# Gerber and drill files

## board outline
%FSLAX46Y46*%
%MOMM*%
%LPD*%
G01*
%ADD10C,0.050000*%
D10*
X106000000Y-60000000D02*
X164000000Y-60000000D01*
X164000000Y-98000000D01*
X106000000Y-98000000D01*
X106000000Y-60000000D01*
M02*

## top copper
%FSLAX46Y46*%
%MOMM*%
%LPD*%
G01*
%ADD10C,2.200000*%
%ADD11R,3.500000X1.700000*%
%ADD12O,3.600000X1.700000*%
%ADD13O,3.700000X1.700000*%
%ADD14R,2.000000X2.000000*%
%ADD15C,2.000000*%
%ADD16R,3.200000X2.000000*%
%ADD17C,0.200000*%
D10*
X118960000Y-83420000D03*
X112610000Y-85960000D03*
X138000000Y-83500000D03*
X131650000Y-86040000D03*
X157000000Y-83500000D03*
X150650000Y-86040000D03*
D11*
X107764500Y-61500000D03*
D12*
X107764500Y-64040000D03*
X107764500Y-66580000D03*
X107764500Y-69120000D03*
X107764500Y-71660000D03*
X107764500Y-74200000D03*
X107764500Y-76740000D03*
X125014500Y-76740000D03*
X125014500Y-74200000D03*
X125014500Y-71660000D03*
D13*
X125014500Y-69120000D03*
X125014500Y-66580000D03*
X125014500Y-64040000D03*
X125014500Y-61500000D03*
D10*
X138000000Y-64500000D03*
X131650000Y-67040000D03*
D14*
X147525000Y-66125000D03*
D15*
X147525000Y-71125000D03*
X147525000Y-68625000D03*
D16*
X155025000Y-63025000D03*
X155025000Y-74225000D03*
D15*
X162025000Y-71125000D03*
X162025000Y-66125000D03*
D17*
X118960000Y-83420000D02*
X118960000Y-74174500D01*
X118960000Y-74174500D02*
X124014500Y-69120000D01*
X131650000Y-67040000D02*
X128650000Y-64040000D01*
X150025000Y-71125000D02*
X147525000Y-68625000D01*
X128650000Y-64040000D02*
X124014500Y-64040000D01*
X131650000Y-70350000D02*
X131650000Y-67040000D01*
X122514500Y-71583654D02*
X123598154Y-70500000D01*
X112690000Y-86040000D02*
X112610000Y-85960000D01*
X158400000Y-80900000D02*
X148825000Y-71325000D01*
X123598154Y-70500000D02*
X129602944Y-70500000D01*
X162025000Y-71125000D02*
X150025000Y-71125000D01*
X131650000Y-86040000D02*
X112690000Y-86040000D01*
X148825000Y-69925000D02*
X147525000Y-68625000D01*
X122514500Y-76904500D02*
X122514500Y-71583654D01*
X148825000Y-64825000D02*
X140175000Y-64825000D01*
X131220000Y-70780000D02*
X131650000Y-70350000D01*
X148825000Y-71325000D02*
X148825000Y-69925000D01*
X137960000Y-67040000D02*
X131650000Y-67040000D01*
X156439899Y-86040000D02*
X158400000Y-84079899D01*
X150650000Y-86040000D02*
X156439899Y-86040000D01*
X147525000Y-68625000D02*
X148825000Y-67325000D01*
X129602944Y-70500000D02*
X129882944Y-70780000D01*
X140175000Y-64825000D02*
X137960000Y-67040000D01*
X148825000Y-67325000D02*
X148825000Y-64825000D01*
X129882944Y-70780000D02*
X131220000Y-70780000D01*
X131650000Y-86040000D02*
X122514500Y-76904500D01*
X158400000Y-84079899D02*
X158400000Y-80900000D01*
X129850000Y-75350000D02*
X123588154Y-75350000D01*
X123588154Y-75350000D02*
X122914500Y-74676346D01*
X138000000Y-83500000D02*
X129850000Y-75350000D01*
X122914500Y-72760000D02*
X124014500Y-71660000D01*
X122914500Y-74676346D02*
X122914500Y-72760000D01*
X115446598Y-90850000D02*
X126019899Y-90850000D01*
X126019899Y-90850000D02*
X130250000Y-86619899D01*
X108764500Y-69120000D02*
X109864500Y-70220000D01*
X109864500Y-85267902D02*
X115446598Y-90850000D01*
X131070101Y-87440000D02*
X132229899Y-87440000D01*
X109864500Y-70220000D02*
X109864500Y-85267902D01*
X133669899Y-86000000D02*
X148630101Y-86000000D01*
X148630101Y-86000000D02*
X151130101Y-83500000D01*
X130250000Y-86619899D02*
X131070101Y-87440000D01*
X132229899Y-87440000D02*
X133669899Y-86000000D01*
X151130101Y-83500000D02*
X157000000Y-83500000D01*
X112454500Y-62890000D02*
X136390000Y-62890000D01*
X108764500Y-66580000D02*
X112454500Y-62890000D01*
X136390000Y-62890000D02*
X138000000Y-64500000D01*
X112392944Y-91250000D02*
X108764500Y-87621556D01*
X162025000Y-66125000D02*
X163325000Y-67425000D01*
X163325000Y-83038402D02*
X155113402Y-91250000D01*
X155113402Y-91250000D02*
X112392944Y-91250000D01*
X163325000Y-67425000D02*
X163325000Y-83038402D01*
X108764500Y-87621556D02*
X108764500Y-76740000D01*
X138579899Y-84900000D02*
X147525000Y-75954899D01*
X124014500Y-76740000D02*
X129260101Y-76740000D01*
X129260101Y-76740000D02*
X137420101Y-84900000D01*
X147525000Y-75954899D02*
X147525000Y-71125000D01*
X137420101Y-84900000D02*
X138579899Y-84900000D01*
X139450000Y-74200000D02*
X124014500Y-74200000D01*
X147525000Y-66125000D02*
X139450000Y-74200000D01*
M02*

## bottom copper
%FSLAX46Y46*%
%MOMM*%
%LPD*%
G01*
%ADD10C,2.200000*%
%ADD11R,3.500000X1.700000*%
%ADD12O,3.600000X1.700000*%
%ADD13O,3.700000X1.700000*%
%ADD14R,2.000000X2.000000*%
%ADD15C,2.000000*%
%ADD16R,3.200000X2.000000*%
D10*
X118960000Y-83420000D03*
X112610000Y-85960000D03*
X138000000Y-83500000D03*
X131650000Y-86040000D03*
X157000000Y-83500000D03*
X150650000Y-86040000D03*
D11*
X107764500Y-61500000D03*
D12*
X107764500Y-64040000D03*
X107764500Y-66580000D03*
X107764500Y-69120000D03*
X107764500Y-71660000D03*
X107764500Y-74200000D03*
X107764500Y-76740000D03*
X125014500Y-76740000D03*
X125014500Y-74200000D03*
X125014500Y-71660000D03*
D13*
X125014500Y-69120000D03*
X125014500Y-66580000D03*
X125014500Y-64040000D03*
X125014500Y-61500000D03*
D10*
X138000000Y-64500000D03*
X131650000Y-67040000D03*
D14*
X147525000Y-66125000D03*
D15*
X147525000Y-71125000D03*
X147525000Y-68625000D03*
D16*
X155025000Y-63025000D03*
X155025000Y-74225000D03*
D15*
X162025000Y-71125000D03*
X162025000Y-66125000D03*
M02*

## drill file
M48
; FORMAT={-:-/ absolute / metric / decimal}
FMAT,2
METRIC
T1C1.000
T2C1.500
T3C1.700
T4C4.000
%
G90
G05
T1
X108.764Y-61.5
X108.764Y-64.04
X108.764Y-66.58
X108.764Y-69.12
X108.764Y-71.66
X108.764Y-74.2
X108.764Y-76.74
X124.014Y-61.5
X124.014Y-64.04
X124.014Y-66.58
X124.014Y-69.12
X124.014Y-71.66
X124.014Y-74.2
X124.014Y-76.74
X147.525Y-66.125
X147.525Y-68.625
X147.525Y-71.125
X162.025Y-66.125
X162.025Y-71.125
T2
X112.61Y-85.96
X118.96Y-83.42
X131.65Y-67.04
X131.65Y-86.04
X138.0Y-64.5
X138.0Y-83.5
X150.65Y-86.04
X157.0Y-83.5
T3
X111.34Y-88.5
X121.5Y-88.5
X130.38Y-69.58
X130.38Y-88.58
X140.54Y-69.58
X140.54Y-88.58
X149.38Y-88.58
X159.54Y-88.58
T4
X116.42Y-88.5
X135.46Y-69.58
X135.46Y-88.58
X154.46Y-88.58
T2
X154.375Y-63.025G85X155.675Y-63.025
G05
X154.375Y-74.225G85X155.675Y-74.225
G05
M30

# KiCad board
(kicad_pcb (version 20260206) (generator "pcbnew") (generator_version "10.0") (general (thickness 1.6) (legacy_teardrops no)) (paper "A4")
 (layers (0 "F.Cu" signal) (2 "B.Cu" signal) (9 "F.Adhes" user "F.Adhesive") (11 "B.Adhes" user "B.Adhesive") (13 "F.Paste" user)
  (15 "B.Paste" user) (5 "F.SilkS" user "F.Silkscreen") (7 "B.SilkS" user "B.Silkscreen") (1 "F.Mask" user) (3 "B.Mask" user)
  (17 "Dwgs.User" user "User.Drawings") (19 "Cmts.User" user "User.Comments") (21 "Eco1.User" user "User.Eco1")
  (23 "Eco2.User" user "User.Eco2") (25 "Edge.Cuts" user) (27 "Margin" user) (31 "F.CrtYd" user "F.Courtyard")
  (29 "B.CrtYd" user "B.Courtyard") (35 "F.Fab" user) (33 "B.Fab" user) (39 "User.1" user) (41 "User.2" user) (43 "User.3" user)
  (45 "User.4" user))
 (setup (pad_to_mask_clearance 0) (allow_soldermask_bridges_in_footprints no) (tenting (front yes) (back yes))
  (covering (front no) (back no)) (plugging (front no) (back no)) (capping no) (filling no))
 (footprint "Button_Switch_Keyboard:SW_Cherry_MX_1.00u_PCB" (layer "F.Cu") (at 118.96 83.42)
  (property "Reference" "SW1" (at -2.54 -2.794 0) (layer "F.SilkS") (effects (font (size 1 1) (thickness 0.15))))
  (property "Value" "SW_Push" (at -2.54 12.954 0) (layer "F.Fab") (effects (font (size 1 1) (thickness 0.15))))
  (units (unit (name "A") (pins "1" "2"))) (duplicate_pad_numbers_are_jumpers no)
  (pad "" np_thru_hole circle (at -7.62 5.08) (size 1.7 1.7) (drill 1.7) (layers "*.Cu" "*.Mask"))
  (pad "" np_thru_hole circle (at -2.54 5.08) (size 4 4) (drill 4) (layers "*.Cu" "*.Mask"))
  (pad "" np_thru_hole circle (at 2.54 5.08) (size 1.7 1.7) (drill 1.7) (layers "*.Cu" "*.Mask"))
  (pad "1" thru_hole circle (at 0 0) (size 2.2 2.2) (drill 1.5) (layers "*.Cu" "*.Mask") (remove_unused_layers no)
   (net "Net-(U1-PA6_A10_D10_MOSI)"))
  (pad "2" thru_hole circle (at -6.35 2.54) (size 2.2 2.2) (drill 1.5) (layers "*.Cu" "*.Mask") (remove_unused_layers no) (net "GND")))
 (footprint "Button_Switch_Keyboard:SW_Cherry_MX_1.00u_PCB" (layer "F.Cu") (at 138 83.5)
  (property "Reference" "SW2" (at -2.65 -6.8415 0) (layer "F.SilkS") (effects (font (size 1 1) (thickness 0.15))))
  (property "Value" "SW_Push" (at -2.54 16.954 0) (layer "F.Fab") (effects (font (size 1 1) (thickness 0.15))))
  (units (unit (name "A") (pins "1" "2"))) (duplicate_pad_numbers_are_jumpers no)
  (pad "" np_thru_hole circle (at -7.62 5.08) (size 1.7 1.7) (drill 1.7) (layers "*.Cu" "*.Mask"))
  (pad "" np_thru_hole circle (at -2.54 5.08) (size 4 4) (drill 4) (layers "*.Cu" "*.Mask"))
  (pad "" np_thru_hole circle (at 2.54 5.08) (size 1.7 1.7) (drill 1.7) (layers "*.Cu" "*.Mask"))
  (pad "1" thru_hole circle (at 0 0) (size 2.2 2.2) (drill 1.5) (layers "*.Cu" "*.Mask") (remove_unused_layers no)
   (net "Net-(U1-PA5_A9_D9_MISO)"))
  (pad "2" thru_hole circle (at -6.35 2.54) (size 2.2 2.2) (drill 1.5) (layers "*.Cu" "*.Mask") (remove_unused_layers no) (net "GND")))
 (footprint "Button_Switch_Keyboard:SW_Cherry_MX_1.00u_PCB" (layer "F.Cu") (at 157 83.5)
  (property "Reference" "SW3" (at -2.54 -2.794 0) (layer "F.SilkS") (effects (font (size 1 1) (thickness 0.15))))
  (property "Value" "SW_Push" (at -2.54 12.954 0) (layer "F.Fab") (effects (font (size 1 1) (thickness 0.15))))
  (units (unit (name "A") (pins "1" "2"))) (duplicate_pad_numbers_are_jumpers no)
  (pad "" np_thru_hole circle (at -7.62 5.08) (size 1.7 1.7) (drill 1.7) (layers "*.Cu" "*.Mask"))
  (pad "" np_thru_hole circle (at -2.54 5.08) (size 4 4) (drill 4) (layers "*.Cu" "*.Mask"))
  (pad "" np_thru_hole circle (at 2.54 5.08) (size 1.7 1.7) (drill 1.7) (layers "*.Cu" "*.Mask"))
  (pad "1" thru_hole circle (at 0 0) (size 2.2 2.2) (drill 1.5) (layers "*.Cu" "*.Mask") (remove_unused_layers no)
   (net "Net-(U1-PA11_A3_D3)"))
  (pad "2" thru_hole circle (at -6.35 2.54) (size 2.2 2.2) (drill 1.5) (layers "*.Cu" "*.Mask") (remove_unused_layers no) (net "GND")))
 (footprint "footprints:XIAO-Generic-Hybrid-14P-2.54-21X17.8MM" (layer "F.Cu") (at 116.3895 69.12)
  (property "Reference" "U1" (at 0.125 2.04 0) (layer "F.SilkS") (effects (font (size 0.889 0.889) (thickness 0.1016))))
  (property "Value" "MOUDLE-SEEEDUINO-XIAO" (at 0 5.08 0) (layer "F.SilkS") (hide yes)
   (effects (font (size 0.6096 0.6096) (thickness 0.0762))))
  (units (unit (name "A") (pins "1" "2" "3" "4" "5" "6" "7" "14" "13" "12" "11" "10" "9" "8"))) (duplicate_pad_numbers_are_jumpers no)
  (pad "1" thru_hole rect (at -7.625 -7.62) (size 3.5 1.7) (drill 1 (offset -1 0)) (layers "*.Cu" "*.Mask") (remove_unused_layers no)
   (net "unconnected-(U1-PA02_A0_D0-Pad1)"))
  (pad "2" thru_hole oval (at -7.625 -5.08) (size 3.6 1.7) (drill 1 (offset -1 0)) (layers "*.Cu" "*.Mask") (remove_unused_layers no)
   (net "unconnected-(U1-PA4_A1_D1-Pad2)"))
  (pad "3" thru_hole oval (at -7.625 -2.54) (size 3.6 1.7) (drill 1 (offset -1 0)) (layers "*.Cu" "*.Mask") (remove_unused_layers no)
   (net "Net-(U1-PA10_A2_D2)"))
  (pad "4" thru_hole oval (at -7.625 0) (size 3.6 1.7) (drill 1 (offset -1 0)) (layers "*.Cu" "*.Mask") (remove_unused_layers no)
   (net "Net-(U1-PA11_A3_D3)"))
  (pad "5" thru_hole oval (at -7.625 2.54) (size 3.6 1.7) (drill 1 (offset -1 0)) (layers "*.Cu" "*.Mask") (remove_unused_layers no)
   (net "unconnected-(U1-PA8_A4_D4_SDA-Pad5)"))
  (pad "6" thru_hole oval (at -7.625 5.08 180) (size 3.6 1.7) (drill 1 (offset 1 0)) (layers "*.Cu" "*.Mask") (remove_unused_layers no)
   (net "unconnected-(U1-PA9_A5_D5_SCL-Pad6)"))
  (pad "7" thru_hole oval (at -7.625 7.62) (size 3.6 1.7) (drill 1 (offset -1 0)) (layers "*.Cu" "*.Mask") (remove_unused_layers no)
   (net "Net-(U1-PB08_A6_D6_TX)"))
  (pad "8" thru_hole oval (at 7.625 7.62) (size 3.6 1.7) (drill 1 (offset 1 0)) (layers "*.Cu" "*.Mask") (remove_unused_layers no)
   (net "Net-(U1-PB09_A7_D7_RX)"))
  (pad "9" thru_hole oval (at 7.625 5.08) (size 3.6 1.7) (drill 1 (offset 1 0)) (layers "*.Cu" "*.Mask") (remove_unused_layers no)
   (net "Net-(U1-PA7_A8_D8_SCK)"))
  (pad "10" thru_hole oval (at 7.625 2.54) (size 3.6 1.7) (drill 1 (offset 1 0)) (layers "*.Cu" "*.Mask") (remove_unused_layers no)
   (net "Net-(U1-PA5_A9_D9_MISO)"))
  (pad "11" thru_hole oval (at 7.625 0) (size 3.7 1.7) (drill 1 (offset 1 0)) (layers "*.Cu" "*.Mask") (remove_unused_layers no)
   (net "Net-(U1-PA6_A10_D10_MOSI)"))
  (pad "12" thru_hole oval (at 7.625 -2.54) (size 3.7 1.7) (drill 1 (offset 1 0)) (layers "*.Cu" "*.Mask") (remove_unused_layers no)
   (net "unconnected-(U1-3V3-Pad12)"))
  (pad "13" thru_hole oval (at 7.625 -5.08) (size 3.7 1.7) (drill 1 (offset 1 0)) (layers "*.Cu" "*.Mask") (remove_unused_layers no)
   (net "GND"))
  (pad "14" thru_hole oval (at 7.625 -7.62) (size 3.7 1.7) (drill 1 (offset 1 0)) (layers "*.Cu" "*.Mask") (remove_unused_layers no)
   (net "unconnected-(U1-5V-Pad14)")))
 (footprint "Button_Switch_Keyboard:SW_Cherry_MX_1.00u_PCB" (layer "F.Cu") (at 138 64.5)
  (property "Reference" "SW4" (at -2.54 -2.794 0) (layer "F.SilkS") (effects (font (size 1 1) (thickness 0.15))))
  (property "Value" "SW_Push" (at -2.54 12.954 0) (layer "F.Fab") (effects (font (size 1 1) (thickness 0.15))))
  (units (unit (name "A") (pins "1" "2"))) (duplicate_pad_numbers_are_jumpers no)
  (pad "" np_thru_hole circle (at -7.62 5.08) (size 1.7 1.7) (drill 1.7) (layers "*.Cu" "*.Mask"))
  (pad "" np_thru_hole circle (at -2.54 5.08) (size 4 4) (drill 4) (layers "*.Cu" "*.Mask"))
  (pad "" np_thru_hole circle (at 2.54 5.08) (size 1.7 1.7) (drill 1.7) (layers "*.Cu" "*.Mask"))
  (pad "1" thru_hole circle (at 0 0) (size 2.2 2.2) (drill 1.5) (layers "*.Cu" "*.Mask") (remove_unused_layers no)
   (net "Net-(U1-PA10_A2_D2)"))
  (pad "2" thru_hole circle (at -6.35 2.54) (size 2.2 2.2) (drill 1.5) (layers "*.Cu" "*.Mask") (remove_unused_layers no) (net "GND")))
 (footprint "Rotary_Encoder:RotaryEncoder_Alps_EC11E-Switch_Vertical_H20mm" (layer "F.Cu") (at 147.525 66.125)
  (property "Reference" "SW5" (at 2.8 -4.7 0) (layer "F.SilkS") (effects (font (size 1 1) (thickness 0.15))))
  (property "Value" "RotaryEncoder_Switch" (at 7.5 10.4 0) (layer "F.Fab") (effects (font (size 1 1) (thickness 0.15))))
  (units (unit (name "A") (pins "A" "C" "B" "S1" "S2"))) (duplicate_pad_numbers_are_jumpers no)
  (pad "A" thru_hole rect (at 0 0) (size 2 2) (drill 1) (layers "*.Cu" "*.Mask") (remove_unused_layers no) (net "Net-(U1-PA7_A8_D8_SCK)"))
  (pad "B" thru_hole circle (at 0 5) (size 2 2) (drill 1) (layers "*.Cu" "*.Mask") (remove_unused_layers no) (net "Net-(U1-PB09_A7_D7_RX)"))
  (pad "C" thru_hole circle (at 0 2.5) (size 2 2) (drill 1) (layers "*.Cu" "*.Mask") (remove_unused_layers no) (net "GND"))
  (pad "MP" thru_hole rect (at 7.5 -3.1) (size 3.2 2) (drill oval 2.8 1.5) (layers "*.Cu" "*.Mask") (remove_unused_layers no))
  (pad "MP" thru_hole rect (at 7.5 8.1) (size 3.2 2) (drill oval 2.8 1.5) (layers "*.Cu" "*.Mask") (remove_unused_layers no))
  (pad "S1" thru_hole circle (at 14.5 5) (size 2 2) (drill 1) (layers "*.Cu" "*.Mask") (remove_unused_layers no) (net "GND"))
  (pad "S2" thru_hole circle (at 14.5 0) (size 2 2) (drill 1) (layers "*.Cu" "*.Mask") (remove_unused_layers no)
   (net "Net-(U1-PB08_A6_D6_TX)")))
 (gr_rect (start 106 60) (end 164 98) (stroke (width 0.05) (type default)) (fill no) (layer "Edge.Cuts"))
 (segment (start 118.96 83.42) (end 118.96 74.1745) (width 0.2) (layer "F.Cu") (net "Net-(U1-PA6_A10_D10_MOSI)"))
 (segment (start 118.96 74.1745) (end 124.0145 69.12) (width 0.2) (layer "F.Cu") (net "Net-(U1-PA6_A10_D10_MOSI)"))
 (segment (start 131.65 67.04) (end 128.65 64.04) (width 0.2) (layer "F.Cu") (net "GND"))
 (segment (start 150.025 71.125) (end 147.525 68.625) (width 0.2) (layer "F.Cu") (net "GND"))
 (segment (start 128.65 64.04) (end 124.0145 64.04) (width 0.2) (layer "F.Cu") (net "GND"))
 (segment (start 131.65 70.35) (end 131.65 67.04) (width 0.2) (layer "F.Cu") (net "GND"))
 (segment (start 122.5145 71.583654) (end 123.598154 70.5) (width 0.2) (layer "F.Cu") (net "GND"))
 (segment (start 112.69 86.04) (end 112.61 85.96) (width 0.2) (layer "F.Cu") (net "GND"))
 (segment (start 158.4 80.9) (end 148.825 71.325) (width 0.2) (layer "F.Cu") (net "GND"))
 (segment (start 123.598154 70.5) (end 129.602944 70.5) (width 0.2) (layer "F.Cu") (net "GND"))
 (segment (start 162.025 71.125) (end 150.025 71.125) (width 0.2) (layer "F.Cu") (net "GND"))
 (segment (start 131.65 86.04) (end 112.69 86.04) (width 0.2) (layer "F.Cu") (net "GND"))
 (segment (start 148.825 69.925) (end 147.525 68.625) (width 0.2) (layer "F.Cu") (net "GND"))
 (segment (start 122.5145 76.9045) (end 122.5145 71.583654) (width 0.2) (layer "F.Cu") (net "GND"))
 (segment (start 148.825 64.825) (end 140.175 64.825) (width 0.2) (layer "F.Cu") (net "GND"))
 (segment (start 131.22 70.78) (end 131.65 70.35) (width 0.2) (layer "F.Cu") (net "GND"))
 (segment (start 148.825 71.325) (end 148.825 69.925) (width 0.2) (layer "F.Cu") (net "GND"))
 (segment (start 137.96 67.04) (end 131.65 67.04) (width 0.2) (layer "F.Cu") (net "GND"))
 (segment (start 156.439899 86.04) (end 158.4 84.079899) (width 0.2) (layer "F.Cu") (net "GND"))
 (segment (start 150.65 86.04) (end 156.439899 86.04) (width 0.2) (layer "F.Cu") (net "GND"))
 (segment (start 147.525 68.625) (end 148.825 67.325) (width 0.2) (layer "F.Cu") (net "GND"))
 (segment (start 129.602944 70.5) (end 129.882944 70.78) (width 0.2) (layer "F.Cu") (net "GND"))
 (segment (start 140.175 64.825) (end 137.96 67.04) (width 0.2) (layer "F.Cu") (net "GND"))
 (segment (start 148.825 67.325) (end 148.825 64.825) (width 0.2) (layer "F.Cu") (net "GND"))
 (segment (start 129.882944 70.78) (end 131.22 70.78) (width 0.2) (layer "F.Cu") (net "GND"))
 (segment (start 131.65 86.04) (end 122.5145 76.9045) (width 0.2) (layer "F.Cu") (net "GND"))
 (segment (start 158.4 84.079899) (end 158.4 80.9) (width 0.2) (layer "F.Cu") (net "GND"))
 (segment (start 129.85 75.35) (end 123.588154 75.35) (width 0.2) (layer "F.Cu") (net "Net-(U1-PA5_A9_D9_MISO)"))
 (segment (start 123.588154 75.35) (end 122.9145 74.676346) (width 0.2) (layer "F.Cu") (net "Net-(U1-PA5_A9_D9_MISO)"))
 (segment (start 138 83.5) (end 129.85 75.35) (width 0.2) (layer "F.Cu") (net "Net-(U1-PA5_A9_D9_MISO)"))
 (segment (start 122.9145 72.76) (end 124.0145 71.66) (width 0.2) (layer "F.Cu") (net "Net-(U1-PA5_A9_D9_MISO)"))
 (segment (start 122.9145 74.676346) (end 122.9145 72.76) (width 0.2) (layer "F.Cu") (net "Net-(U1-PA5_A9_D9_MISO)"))
 (segment (start 115.446598 90.85) (end 126.019899 90.85) (width 0.2) (layer "F.Cu") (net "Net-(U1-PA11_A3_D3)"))
 (segment (start 126.019899 90.85) (end 130.25 86.619899) (width 0.2) (layer "F.Cu") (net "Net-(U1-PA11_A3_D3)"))
 (segment (start 108.7645 69.12) (end 109.8645 70.22) (width 0.2) (layer "F.Cu") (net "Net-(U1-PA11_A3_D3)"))
 (segment (start 109.8645 85.267902) (end 115.446598 90.85) (width 0.2) (layer "F.Cu") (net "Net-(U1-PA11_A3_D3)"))
 (segment (start 131.070101 87.44) (end 132.229899 87.44) (width 0.2) (layer "F.Cu") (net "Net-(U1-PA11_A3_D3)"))
 (segment (start 109.8645 70.22) (end 109.8645 85.267902) (width 0.2) (layer "F.Cu") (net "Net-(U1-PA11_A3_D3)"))
 (segment (start 133.669899 86) (end 148.630101 86) (width 0.2) (layer "F.Cu") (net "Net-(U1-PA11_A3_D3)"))
 (segment (start 148.630101 86) (end 151.130101 83.5) (width 0.2) (layer "F.Cu") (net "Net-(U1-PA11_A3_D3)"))
 (segment (start 130.25 86.619899) (end 131.070101 87.44) (width 0.2) (layer "F.Cu") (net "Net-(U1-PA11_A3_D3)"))
 (segment (start 132.229899 87.44) (end 133.669899 86) (width 0.2) (layer "F.Cu") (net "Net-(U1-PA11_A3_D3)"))
 (segment (start 151.130101 83.5) (end 157 83.5) (width 0.2) (layer "F.Cu") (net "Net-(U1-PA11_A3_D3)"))
 (segment (start 112.4545 62.89) (end 136.39 62.89) (width 0.2) (layer "F.Cu") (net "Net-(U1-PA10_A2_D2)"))
 (segment (start 108.7645 66.58) (end 112.4545 62.89) (width 0.2) (layer "F.Cu") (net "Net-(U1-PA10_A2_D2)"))
 (segment (start 136.39 62.89) (end 138 64.5) (width 0.2) (layer "F.Cu") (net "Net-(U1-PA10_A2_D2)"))
 (segment (start 112.392944 91.25) (end 108.7645 87.621556) (width 0.2) (layer "F.Cu") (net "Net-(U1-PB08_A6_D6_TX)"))
 (segment (start 162.025 66.125) (end 163.325 67.425) (width 0.2) (layer "F.Cu") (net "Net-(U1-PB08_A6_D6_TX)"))
 (segment (start 163.325 83.038402) (end 155.113402 91.25) (width 0.2) (layer "F.Cu") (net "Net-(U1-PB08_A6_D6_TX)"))
 (segment (start 155.113402 91.25) (end 112.392944 91.25) (width 0.2) (layer "F.Cu") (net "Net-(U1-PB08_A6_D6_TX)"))
 (segment (start 163.325 67.425) (end 163.325 83.038402) (width 0.2) (layer "F.Cu") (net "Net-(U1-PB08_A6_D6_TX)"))
 (segment (start 108.7645 87.621556) (end 108.7645 76.74) (width 0.2) (layer "F.Cu") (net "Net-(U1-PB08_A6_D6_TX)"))
 (segment (start 138.579899 84.9) (end 147.525 75.954899) (width 0.2) (layer "F.Cu") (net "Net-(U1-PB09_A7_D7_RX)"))
 (segment (start 124.0145 76.74) (end 129.260101 76.74) (width 0.2) (layer "F.Cu") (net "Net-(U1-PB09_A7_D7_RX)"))
 (segment (start 129.260101 76.74) (end 137.420101 84.9) (width 0.2) (layer "F.Cu") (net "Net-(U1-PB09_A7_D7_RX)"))
 (segment (start 147.525 75.954899) (end 147.525 71.125) (width 0.2) (layer "F.Cu") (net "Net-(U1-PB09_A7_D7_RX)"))
 (segment (start 137.420101 84.9) (end 138.579899 84.9) (width 0.2) (layer "F.Cu") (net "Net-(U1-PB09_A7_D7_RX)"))
 (segment (start 139.45 74.2) (end 124.0145 74.2) (width 0.2) (layer "F.Cu") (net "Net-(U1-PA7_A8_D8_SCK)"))
 (segment (start 147.525 66.125) (end 139.45 74.2) (width 0.2) (layer "F.Cu") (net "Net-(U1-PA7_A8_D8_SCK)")))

